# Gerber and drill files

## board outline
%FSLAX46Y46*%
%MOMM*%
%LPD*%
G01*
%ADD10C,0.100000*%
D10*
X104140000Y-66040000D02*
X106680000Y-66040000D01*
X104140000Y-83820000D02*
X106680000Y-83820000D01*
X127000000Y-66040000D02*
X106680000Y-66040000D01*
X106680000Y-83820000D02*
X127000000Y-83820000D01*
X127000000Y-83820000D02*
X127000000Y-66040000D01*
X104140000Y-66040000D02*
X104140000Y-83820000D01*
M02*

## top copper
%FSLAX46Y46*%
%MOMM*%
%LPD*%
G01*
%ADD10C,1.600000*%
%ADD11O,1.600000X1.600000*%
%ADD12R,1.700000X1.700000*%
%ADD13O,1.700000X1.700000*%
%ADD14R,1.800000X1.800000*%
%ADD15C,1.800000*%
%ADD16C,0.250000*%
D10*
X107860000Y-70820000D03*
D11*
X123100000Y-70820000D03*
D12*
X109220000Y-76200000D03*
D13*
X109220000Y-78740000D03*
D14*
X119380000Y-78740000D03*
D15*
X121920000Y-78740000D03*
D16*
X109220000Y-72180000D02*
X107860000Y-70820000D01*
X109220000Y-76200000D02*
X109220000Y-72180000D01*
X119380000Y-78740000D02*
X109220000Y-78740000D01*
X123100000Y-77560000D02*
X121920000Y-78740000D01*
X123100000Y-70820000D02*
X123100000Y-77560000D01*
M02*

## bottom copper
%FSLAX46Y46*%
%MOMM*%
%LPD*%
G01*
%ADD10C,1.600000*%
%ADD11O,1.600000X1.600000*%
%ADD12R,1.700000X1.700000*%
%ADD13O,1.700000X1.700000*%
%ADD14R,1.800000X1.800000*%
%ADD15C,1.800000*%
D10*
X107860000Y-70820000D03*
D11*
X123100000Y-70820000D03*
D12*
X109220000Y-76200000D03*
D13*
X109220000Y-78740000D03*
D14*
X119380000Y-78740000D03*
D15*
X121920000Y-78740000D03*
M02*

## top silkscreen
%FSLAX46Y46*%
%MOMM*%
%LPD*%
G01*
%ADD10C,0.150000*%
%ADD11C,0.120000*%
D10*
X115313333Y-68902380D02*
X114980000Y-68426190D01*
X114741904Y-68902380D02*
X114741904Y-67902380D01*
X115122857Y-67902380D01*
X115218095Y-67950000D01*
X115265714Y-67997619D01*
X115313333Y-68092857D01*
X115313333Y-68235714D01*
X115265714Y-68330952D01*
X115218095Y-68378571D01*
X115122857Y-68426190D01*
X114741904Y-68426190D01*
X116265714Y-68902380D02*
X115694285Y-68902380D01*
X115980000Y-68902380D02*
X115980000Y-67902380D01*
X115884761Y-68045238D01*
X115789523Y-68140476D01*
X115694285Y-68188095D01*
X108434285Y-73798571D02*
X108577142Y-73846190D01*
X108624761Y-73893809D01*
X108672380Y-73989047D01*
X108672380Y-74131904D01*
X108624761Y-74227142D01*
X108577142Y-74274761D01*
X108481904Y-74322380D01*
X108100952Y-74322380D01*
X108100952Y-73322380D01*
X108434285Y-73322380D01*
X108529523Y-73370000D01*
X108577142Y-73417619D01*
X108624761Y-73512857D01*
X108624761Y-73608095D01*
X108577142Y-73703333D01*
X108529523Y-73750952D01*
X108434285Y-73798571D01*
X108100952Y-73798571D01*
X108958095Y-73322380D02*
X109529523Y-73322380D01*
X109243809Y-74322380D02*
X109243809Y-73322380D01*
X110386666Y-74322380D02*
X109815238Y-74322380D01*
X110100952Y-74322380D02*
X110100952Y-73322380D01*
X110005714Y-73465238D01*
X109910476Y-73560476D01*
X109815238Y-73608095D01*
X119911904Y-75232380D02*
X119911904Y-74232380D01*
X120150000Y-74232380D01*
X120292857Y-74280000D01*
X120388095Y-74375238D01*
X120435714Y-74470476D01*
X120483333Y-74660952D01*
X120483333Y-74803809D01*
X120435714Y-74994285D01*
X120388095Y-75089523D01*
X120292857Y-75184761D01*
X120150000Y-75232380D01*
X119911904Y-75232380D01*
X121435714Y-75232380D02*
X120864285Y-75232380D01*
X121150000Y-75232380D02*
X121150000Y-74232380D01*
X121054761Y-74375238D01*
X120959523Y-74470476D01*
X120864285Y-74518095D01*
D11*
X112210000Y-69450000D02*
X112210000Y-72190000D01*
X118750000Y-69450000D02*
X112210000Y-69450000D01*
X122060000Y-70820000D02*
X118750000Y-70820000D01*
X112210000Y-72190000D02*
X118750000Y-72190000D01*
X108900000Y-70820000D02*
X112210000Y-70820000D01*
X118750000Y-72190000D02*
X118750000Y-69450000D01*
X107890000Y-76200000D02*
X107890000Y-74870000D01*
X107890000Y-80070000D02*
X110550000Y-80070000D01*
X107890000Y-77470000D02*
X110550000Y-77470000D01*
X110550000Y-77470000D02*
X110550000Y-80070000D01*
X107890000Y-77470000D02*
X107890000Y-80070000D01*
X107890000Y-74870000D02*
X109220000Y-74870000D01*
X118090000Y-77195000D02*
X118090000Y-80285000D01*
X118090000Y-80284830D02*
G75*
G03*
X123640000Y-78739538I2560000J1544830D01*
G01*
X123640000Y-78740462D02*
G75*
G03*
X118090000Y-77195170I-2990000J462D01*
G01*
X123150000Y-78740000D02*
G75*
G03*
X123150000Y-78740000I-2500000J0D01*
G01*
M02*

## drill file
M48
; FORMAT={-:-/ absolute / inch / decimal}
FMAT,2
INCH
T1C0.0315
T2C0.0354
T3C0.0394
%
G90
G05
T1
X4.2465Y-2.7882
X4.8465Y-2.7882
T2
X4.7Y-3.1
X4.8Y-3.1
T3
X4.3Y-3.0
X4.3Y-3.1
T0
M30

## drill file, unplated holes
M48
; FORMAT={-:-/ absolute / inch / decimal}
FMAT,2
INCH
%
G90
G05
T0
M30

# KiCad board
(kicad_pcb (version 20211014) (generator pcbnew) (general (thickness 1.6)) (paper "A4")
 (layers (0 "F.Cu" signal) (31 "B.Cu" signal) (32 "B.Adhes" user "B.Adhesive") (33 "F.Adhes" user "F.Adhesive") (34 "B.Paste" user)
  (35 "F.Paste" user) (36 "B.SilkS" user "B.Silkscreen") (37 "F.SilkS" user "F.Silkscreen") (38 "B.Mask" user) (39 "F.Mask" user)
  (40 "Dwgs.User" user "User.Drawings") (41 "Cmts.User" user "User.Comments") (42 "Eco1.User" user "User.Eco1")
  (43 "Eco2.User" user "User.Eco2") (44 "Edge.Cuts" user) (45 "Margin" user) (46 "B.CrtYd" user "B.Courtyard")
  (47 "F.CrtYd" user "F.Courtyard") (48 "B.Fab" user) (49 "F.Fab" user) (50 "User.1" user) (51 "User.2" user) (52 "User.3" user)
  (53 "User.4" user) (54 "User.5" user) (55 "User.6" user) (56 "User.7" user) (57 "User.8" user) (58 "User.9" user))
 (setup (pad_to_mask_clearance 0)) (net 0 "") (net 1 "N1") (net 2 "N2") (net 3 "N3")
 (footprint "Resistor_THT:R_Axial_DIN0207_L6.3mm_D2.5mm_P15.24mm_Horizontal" (layer "F.Cu") (at 107.86 70.82)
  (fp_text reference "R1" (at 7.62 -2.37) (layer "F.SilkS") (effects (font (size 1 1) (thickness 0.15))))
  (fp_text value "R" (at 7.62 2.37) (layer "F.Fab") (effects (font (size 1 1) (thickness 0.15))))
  (fp_line (start 4.35 -1.37) (end 4.35 1.37) (layer "F.SilkS") (width 0.12))
  (fp_line (start 10.89 -1.37) (end 4.35 -1.37) (layer "F.SilkS") (width 0.12))
  (fp_line (start 14.2 0) (end 10.89 0) (layer "F.SilkS") (width 0.12))
  (fp_line (start 4.35 1.37) (end 10.89 1.37) (layer "F.SilkS") (width 0.12))
  (fp_line (start 1.04 0) (end 4.35 0) (layer "F.SilkS") (width 0.12))
  (fp_line (start 10.89 1.37) (end 10.89 -1.37) (layer "F.SilkS") (width 0.12))
  (pad "1" thru_hole circle (at 0 0) (size 1.6 1.6) (drill 0.8) (layers *.Cu *.Mask) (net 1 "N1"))
  (pad "2" thru_hole oval (at 15.24 0) (size 1.6 1.6) (drill 0.8) (layers *.Cu *.Mask) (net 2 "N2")))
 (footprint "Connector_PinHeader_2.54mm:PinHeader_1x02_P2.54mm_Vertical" (layer "F.Cu") (at 109.22 76.2)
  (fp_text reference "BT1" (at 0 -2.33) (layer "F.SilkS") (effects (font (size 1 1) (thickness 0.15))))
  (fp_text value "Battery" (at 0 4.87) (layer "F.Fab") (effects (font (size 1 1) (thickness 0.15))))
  (fp_line (start -1.33 0) (end -1.33 -1.33) (layer "F.SilkS") (width 0.12))
  (fp_line (start -1.33 3.87) (end 1.33 3.87) (layer "F.SilkS") (width 0.12))
  (fp_line (start -1.33 1.27) (end 1.33 1.27) (layer "F.SilkS") (width 0.12))
  (fp_line (start 1.33 1.27) (end 1.33 3.87) (layer "F.SilkS") (width 0.12))
  (fp_line (start -1.33 1.27) (end -1.33 3.87) (layer "F.SilkS") (width 0.12))
  (fp_line (start -1.33 -1.33) (end 0 -1.33) (layer "F.SilkS") (width 0.12))
  (pad "1" thru_hole rect (at 0 0) (size 1.7 1.7) (drill 1) (layers *.Cu *.Mask) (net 1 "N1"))
  (pad "2" thru_hole oval (at 0 2.54) (size 1.7 1.7) (drill 1) (layers *.Cu *.Mask) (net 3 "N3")))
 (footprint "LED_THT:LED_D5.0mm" (layer "F.Cu") (at 119.38 78.74)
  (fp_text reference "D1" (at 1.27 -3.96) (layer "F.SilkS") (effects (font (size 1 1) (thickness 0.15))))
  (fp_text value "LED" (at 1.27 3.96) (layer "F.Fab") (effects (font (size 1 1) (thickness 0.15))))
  (fp_line (start -1.29 -1.545) (end -1.29 1.545) (layer "F.SilkS") (width 0.12))
  (fp_arc (start 4.26 -0.000462) (mid 2.072002 2.880433) (end -1.29 1.54483) (layer "F.SilkS") (width 0.12))
  (fp_arc (start -1.29 -1.54483) (mid 2.072002 -2.880433) (end 4.26 0.000462) (layer "F.SilkS") (width 0.12))
  (fp_circle (center 1.27 0) (end 3.77 0) (layer "F.SilkS") (width 0.12) (fill none))
  (pad "1" thru_hole rect (at 0 0) (size 1.8 1.8) (drill 0.9) (layers *.Cu *.Mask) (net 3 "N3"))
  (pad "2" thru_hole circle (at 2.54 0) (size 1.8 1.8) (drill 0.9) (layers *.Cu *.Mask) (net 2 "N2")))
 (gr_line (start 127 66.04) (end 106.68 66.04) (layer "Edge.Cuts") (width 0.1))
 (gr_line (start 104.14 83.82) (end 106.68 83.82) (layer "Edge.Cuts") (width 0.1))
 (gr_line (start 104.14 66.04) (end 106.68 66.04) (layer "Edge.Cuts") (width 0.1))
 (gr_line (start 106.68 83.82) (end 127 83.82) (layer "Edge.Cuts") (width 0.1))
 (gr_line (start 127 83.82) (end 127 66.04) (layer "Edge.Cuts") (width 0.1))
 (gr_line (start 104.14 66.04) (end 104.14 83.82) (layer "Edge.Cuts") (width 0.1))
 (segment (start 109.22 72.18) (end 107.86 70.82) (width 0.25) (layer "F.Cu") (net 1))
 (segment (start 109.22 76.2) (end 109.22 72.18) (width 0.25) (layer "F.Cu") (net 1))
 (segment (start 119.38 78.74) (end 109.22 78.74) (width 0.25) (layer "F.Cu") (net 3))
 (segment (start 123.1 77.56) (end 121.92 78.74) (width 0.25) (layer "F.Cu") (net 2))
 (segment (start 123.1 70.82) (end 123.1 77.56) (width 0.25) (layer "F.Cu") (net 2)))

